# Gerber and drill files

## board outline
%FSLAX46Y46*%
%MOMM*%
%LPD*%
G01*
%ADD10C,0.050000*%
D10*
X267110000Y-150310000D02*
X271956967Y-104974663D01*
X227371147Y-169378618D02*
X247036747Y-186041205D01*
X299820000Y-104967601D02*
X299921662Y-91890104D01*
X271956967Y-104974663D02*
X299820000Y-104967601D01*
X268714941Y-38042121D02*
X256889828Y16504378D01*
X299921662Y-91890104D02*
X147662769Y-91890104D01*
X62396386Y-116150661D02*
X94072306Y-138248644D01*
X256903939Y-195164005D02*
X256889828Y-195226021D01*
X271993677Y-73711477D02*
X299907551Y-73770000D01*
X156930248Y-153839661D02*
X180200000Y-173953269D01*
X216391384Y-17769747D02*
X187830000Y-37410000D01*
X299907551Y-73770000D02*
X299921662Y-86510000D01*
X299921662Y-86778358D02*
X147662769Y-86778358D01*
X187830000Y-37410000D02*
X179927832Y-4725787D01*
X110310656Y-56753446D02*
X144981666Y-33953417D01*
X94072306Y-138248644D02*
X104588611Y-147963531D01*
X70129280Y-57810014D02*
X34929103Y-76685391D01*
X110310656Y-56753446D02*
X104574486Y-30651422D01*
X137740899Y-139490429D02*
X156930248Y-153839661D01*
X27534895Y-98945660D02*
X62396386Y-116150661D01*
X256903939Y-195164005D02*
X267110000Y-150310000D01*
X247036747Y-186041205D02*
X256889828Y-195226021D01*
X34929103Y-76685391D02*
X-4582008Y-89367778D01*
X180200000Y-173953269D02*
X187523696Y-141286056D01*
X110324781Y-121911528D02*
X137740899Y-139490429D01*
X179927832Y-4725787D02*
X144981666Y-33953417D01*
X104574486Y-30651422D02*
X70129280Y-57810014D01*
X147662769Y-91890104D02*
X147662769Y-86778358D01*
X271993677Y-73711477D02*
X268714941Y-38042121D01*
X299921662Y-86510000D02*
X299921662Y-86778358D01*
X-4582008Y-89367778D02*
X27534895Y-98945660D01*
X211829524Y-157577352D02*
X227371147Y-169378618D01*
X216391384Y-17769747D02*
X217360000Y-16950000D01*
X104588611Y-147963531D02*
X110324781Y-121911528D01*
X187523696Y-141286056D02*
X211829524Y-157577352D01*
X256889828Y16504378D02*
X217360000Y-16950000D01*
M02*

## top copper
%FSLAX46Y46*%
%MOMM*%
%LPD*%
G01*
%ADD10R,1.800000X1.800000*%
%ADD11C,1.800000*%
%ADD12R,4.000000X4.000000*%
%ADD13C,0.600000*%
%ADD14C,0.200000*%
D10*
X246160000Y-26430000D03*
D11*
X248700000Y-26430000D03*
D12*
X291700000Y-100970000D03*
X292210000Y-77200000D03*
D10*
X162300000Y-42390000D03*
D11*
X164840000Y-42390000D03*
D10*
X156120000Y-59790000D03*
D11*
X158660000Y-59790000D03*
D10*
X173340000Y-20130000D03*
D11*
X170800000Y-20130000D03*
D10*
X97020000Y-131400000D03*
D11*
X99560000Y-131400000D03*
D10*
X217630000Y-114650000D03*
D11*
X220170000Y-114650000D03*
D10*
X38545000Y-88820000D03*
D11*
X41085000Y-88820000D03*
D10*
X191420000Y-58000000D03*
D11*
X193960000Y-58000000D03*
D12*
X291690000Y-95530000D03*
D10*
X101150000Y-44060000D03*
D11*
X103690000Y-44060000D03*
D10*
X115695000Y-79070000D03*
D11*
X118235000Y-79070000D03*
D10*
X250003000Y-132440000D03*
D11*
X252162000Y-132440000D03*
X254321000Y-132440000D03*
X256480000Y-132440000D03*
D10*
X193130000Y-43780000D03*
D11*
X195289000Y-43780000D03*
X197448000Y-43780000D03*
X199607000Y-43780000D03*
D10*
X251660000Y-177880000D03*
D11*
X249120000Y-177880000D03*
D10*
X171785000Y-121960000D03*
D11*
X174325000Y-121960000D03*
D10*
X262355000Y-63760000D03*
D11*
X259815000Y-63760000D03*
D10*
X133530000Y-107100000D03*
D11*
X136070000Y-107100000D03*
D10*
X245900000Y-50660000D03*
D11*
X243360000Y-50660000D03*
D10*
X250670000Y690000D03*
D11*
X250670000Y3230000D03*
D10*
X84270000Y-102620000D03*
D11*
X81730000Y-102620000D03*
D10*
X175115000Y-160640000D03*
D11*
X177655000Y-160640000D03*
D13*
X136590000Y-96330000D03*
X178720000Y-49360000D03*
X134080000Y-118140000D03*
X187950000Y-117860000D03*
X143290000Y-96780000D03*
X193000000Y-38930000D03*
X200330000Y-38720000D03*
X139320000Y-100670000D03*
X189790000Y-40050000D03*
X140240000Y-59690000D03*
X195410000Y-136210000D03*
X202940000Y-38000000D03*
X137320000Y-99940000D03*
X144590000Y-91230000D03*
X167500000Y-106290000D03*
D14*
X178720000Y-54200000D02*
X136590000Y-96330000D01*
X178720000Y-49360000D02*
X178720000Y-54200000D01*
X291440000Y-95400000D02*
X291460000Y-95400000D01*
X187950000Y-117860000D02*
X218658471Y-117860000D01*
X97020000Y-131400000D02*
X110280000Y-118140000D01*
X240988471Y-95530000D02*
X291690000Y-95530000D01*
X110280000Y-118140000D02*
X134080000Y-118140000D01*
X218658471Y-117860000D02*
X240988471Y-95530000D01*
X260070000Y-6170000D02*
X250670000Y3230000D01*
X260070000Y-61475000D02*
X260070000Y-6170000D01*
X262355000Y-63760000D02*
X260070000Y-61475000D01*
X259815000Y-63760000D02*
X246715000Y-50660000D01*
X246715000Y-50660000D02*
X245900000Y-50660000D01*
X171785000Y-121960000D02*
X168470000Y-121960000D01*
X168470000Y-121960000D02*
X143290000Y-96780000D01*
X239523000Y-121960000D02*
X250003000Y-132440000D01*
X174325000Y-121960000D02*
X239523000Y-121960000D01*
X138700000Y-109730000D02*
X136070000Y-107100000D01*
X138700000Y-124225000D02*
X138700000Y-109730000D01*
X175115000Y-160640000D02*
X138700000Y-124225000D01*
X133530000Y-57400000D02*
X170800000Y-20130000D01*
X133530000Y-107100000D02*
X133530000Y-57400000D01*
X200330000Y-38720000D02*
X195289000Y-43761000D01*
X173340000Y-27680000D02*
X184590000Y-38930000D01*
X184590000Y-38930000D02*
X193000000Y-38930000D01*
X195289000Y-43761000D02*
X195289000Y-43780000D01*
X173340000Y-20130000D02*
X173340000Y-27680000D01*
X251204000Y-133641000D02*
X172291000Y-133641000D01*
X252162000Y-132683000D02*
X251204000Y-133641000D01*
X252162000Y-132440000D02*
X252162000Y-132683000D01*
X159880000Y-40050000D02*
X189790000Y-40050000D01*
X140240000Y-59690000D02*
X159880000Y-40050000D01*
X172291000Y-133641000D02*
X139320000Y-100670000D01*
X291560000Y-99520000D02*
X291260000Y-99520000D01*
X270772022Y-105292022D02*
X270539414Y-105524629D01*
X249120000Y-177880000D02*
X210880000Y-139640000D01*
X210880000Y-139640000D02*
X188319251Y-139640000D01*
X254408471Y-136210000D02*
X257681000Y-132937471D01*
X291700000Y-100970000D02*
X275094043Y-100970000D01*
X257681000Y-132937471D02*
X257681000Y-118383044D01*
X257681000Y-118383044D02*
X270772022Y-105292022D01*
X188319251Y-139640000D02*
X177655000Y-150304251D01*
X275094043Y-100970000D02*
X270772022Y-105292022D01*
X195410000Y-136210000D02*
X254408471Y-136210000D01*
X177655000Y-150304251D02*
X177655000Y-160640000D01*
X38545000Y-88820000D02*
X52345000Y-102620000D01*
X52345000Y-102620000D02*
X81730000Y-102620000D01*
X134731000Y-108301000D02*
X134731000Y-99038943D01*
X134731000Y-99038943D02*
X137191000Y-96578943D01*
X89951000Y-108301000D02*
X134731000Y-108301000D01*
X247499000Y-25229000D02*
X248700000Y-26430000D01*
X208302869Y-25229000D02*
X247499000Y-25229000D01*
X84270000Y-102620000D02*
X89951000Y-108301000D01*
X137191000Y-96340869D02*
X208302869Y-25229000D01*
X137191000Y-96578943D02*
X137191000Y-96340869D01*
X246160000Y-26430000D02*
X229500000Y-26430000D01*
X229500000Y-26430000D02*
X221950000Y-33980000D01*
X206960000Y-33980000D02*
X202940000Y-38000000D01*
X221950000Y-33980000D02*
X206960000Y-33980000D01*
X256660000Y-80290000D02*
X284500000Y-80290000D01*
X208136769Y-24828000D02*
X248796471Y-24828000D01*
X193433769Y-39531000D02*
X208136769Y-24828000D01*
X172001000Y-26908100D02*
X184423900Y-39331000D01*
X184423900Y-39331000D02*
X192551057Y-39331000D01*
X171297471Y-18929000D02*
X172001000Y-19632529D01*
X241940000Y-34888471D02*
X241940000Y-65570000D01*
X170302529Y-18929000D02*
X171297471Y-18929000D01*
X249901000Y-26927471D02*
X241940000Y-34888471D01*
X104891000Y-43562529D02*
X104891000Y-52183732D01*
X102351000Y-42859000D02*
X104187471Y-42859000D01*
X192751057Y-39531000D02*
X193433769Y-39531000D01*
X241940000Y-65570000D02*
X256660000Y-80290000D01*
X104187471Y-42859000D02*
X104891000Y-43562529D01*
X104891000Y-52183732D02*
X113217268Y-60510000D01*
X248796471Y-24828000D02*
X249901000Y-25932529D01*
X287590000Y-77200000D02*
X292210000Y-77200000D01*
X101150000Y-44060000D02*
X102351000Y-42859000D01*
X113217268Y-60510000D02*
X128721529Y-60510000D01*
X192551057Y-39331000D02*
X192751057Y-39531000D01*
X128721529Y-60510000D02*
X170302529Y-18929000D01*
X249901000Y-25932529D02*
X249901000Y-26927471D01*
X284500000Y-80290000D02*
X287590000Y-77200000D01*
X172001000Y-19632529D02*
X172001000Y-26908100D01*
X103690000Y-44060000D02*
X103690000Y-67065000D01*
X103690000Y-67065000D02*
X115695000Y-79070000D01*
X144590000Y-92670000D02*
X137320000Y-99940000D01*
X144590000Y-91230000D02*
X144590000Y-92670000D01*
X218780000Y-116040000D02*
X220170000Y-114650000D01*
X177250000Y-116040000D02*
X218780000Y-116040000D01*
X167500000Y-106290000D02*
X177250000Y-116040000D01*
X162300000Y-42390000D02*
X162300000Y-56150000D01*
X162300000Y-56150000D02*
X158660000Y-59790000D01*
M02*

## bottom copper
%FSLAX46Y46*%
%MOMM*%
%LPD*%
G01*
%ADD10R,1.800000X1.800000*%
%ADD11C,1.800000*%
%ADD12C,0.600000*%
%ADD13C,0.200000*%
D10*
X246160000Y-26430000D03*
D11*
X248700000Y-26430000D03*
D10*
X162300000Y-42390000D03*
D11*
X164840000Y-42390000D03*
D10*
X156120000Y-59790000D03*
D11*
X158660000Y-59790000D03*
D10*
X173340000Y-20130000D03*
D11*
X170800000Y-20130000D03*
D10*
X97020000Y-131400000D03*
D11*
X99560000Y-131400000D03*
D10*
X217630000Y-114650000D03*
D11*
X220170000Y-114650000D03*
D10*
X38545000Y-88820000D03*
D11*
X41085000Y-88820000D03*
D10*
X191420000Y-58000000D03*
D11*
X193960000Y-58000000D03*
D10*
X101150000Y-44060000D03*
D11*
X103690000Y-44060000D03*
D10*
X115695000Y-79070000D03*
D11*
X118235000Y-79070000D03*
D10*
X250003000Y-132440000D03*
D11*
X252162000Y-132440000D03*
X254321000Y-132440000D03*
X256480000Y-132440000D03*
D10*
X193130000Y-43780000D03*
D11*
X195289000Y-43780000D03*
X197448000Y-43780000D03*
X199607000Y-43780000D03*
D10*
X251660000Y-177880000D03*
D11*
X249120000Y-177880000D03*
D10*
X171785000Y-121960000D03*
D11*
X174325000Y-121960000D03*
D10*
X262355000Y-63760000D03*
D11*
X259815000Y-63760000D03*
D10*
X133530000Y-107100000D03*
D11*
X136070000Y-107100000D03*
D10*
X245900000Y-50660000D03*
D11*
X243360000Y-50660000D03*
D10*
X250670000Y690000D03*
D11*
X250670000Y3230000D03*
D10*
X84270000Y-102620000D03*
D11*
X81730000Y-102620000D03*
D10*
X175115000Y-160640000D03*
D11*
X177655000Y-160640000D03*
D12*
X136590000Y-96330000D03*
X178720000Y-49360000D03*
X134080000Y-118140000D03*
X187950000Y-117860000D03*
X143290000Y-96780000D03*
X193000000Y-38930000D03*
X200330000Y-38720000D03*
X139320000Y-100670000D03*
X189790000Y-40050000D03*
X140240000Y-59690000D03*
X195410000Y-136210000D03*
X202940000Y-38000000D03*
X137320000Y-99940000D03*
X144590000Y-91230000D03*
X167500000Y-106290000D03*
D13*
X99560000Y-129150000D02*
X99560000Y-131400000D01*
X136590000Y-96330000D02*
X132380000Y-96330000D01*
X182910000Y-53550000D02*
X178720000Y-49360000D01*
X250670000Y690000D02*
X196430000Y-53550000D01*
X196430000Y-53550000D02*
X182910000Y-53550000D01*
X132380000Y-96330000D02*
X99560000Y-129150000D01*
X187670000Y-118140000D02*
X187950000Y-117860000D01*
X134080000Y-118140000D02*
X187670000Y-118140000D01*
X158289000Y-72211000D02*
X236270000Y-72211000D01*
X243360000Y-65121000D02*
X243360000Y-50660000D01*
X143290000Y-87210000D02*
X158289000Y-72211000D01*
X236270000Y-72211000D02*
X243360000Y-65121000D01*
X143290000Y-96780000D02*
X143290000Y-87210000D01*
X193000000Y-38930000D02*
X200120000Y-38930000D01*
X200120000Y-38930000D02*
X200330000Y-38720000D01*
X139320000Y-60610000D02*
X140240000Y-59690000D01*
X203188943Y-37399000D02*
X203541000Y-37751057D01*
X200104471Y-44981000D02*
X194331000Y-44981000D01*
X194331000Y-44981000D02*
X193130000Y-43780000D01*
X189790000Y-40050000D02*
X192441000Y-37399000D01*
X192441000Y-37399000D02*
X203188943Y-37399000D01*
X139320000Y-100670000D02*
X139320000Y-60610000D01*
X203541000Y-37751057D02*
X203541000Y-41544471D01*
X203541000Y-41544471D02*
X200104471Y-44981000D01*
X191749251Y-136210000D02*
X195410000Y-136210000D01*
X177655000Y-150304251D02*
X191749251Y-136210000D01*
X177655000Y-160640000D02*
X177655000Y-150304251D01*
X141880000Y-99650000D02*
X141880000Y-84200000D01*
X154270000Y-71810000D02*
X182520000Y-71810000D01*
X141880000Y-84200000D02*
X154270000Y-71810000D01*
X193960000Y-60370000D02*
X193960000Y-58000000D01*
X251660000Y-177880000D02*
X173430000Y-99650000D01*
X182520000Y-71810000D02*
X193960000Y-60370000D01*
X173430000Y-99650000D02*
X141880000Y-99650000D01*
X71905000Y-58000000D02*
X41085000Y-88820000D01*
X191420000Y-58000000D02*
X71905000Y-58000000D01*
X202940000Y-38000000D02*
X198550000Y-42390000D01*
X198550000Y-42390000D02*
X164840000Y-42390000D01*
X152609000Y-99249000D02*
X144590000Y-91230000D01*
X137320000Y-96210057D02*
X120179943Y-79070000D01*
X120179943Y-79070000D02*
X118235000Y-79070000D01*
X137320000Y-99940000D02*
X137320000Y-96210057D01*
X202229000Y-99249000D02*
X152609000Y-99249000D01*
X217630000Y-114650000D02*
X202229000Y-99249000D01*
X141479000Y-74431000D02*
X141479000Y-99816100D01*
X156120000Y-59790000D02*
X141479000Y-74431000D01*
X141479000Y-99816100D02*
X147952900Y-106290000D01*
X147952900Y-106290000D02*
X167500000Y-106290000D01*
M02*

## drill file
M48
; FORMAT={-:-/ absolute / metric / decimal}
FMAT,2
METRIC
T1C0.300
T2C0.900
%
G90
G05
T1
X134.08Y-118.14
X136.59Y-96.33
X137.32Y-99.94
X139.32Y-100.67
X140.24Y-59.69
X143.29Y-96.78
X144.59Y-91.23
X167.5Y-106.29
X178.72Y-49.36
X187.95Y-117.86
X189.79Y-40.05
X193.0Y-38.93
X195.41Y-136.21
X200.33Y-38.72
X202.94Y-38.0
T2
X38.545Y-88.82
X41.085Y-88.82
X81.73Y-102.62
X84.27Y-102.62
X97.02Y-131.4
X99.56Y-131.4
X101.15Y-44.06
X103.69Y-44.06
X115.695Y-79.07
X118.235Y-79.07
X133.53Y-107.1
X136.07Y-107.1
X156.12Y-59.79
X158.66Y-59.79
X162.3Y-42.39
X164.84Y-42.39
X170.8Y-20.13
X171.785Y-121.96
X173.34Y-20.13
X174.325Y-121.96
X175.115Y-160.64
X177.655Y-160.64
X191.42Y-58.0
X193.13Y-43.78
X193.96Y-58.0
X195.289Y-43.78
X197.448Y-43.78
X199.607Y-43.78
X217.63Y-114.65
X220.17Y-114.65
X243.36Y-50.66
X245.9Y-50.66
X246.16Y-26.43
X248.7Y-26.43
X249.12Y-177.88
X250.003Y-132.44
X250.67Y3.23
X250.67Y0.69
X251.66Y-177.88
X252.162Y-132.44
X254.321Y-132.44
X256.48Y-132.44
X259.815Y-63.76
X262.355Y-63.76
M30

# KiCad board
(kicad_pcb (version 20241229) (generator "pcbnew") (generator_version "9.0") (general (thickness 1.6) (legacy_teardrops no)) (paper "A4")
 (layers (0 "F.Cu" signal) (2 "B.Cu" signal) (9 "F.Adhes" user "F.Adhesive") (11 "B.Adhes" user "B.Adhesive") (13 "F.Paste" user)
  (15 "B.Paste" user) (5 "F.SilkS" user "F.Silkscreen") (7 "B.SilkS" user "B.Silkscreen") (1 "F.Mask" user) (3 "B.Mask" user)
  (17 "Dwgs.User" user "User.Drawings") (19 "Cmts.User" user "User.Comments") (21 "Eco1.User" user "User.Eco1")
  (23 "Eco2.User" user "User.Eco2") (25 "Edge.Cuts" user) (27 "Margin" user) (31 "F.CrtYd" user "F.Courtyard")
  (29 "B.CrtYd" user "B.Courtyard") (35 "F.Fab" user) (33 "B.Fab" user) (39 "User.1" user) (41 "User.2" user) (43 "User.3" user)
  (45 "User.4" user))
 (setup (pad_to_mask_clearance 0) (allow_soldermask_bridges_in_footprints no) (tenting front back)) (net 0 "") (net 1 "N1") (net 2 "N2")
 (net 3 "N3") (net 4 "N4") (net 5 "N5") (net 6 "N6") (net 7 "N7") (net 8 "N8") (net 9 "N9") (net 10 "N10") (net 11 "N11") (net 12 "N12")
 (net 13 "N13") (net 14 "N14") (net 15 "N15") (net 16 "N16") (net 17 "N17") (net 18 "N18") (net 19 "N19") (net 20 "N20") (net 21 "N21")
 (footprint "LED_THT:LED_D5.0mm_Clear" (layer "F.Cu") (at 246.16 26.43)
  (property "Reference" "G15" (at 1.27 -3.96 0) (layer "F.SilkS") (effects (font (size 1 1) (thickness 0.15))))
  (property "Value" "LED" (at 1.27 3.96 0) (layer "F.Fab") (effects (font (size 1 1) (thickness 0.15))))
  (pad "1" thru_hole rect (at 0 0) (size 1.8 1.8) (drill 0.9) (layers "*.Cu" "*.Mask") (remove_unused_layers no) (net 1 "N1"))
  (pad "2" thru_hole circle (at 2.54 0) (size 1.8 1.8) (drill 0.9) (layers "*.Cu" "*.Mask") (remove_unused_layers no) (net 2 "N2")))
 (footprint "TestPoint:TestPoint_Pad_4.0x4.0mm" (layer "F.Cu") (at 291.7 100.97)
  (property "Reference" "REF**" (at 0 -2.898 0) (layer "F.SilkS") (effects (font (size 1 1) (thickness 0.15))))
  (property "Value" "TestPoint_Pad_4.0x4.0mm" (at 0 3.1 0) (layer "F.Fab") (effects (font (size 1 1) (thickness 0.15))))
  (pad "1" smd rect (at 0 0) (size 4 4) (layers "F.Cu" "F.Mask") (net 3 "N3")))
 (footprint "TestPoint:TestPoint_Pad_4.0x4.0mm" (layer "F.Cu") (at 292.21 77.2)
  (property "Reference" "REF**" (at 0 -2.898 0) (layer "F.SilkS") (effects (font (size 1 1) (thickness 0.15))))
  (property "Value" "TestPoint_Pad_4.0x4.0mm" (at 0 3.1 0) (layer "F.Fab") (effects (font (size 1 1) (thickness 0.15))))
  (pad "1" smd rect (at 0 0) (size 4 4) (layers "F.Cu" "F.Mask") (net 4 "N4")))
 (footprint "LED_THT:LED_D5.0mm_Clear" (layer "F.Cu") (at 162.3 42.39)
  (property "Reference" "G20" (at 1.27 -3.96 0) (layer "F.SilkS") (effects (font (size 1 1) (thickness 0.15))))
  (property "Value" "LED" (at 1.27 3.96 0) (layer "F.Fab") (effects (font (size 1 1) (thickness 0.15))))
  (pad "1" thru_hole rect (at 0 0) (size 1.8 1.8) (drill 0.9) (layers "*.Cu" "*.Mask") (remove_unused_layers no) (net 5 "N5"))
  (pad "2" thru_hole circle (at 2.54 0) (size 1.8 1.8) (drill 0.9) (layers "*.Cu" "*.Mask") (remove_unused_layers no) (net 1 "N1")))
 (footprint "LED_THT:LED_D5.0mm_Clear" (layer "F.Cu") (at 156.12 59.79)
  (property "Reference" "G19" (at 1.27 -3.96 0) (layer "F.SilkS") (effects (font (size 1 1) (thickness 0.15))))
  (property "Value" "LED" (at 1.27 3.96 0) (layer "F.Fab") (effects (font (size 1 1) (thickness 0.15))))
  (pad "1" thru_hole rect (at 0 0) (size 1.8 1.8) (drill 0.9) (layers "*.Cu" "*.Mask") (remove_unused_layers no) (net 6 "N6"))
  (pad "2" thru_hole circle (at 2.54 0) (size 1.8 1.8) (drill 0.9) (layers "*.Cu" "*.Mask") (remove_unused_layers no) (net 5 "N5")))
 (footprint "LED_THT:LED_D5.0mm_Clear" (layer "F.Cu") (at 173.34 20.13 180)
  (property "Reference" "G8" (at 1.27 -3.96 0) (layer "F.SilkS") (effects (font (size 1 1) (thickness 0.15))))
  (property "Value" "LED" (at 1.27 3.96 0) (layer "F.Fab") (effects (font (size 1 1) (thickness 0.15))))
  (pad "1" thru_hole rect (at 0 0 180) (size 1.8 1.8) (drill 0.9) (layers "*.Cu" "*.Mask") (remove_unused_layers no) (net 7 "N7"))
  (pad "2" thru_hole circle (at 2.54 0 180) (size 1.8 1.8) (drill 0.9) (layers "*.Cu" "*.Mask") (remove_unused_layers no) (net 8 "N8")))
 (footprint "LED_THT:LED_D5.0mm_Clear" (layer "F.Cu") (at 97.02 131.4)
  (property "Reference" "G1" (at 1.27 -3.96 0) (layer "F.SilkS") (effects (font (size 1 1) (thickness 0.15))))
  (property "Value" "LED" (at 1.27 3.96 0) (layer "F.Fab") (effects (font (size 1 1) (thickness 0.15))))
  (pad "1" thru_hole rect (at 0 0) (size 1.8 1.8) (drill 0.9) (layers "*.Cu" "*.Mask") (remove_unused_layers no) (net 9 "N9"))
  (pad "2" thru_hole circle (at 2.54 0) (size 1.8 1.8) (drill 0.9) (layers "*.Cu" "*.Mask") (remove_unused_layers no) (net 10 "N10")))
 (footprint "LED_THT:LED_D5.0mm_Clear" (layer "F.Cu") (at 217.63 114.65)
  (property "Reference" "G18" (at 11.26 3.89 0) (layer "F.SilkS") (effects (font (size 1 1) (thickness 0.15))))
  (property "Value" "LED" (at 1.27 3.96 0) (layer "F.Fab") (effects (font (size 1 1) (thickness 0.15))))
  (pad "1" thru_hole rect (at 0 0) (size 1.8 1.8) (drill 0.9) (layers "*.Cu" "*.Mask") (remove_unused_layers no) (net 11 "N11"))
  (pad "2" thru_hole circle (at 2.54 0) (size 1.8 1.8) (drill 0.9) (layers "*.Cu" "*.Mask") (remove_unused_layers no) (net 6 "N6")))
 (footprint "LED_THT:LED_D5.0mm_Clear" (layer "F.Cu") (at 38.545 88.82)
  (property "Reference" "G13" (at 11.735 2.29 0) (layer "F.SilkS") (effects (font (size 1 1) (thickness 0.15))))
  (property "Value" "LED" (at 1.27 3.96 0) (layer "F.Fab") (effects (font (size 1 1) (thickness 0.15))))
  (pad "1" thru_hole rect (at 0 0) (size 1.8 1.8) (drill 0.9) (layers "*.Cu" "*.Mask") (remove_unused_layers no) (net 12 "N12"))
  (pad "2" thru_hole circle (at 2.54 0) (size 1.8 1.8) (drill 0.9) (layers "*.Cu" "*.Mask") (remove_unused_layers no) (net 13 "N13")))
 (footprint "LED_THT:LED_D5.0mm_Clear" (layer "F.Cu") (at 191.42 58)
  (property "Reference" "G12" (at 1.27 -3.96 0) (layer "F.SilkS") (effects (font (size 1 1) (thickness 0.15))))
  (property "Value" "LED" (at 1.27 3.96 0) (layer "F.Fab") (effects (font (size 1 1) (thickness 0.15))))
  (pad "1" thru_hole rect (at 0 0) (size 1.8 1.8) (drill 0.9) (layers "*.Cu" "*.Mask") (remove_unused_layers no) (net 13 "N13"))
  (pad "2" thru_hole circle (at 2.54 0) (size 1.8 1.8) (drill 0.9) (layers "*.Cu" "*.Mask") (remove_unused_layers no) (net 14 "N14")))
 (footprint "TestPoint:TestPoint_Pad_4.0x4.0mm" (layer "F.Cu") (at 291.69 95.53)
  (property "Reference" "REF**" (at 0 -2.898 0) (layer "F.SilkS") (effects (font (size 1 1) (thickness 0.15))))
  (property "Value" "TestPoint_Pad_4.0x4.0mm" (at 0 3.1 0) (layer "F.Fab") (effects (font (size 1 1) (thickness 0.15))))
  (pad "1" smd rect (at 0 0) (size 4 4) (layers "F.Cu" "F.Mask") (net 9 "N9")))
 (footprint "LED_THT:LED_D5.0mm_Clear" (layer "F.Cu") (at 101.15 44.06)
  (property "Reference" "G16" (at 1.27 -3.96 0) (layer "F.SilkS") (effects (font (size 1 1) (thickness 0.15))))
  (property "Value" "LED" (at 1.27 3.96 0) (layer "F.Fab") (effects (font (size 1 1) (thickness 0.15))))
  (pad "1" thru_hole rect (at 0 0) (size 1.8 1.8) (drill 0.9) (layers "*.Cu" "*.Mask") (remove_unused_layers no) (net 4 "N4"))
  (pad "2" thru_hole circle (at 2.54 0) (size 1.8 1.8) (drill 0.9) (layers "*.Cu" "*.Mask") (remove_unused_layers no) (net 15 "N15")))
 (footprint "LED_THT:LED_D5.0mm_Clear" (layer "F.Cu") (at 115.695 79.07)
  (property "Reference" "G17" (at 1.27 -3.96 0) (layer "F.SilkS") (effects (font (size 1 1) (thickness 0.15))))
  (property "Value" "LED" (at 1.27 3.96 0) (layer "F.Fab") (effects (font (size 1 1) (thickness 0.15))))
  (pad "1" thru_hole rect (at 0 0) (size 1.8 1.8) (drill 0.9) (layers "*.Cu" "*.Mask") (remove_unused_layers no) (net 15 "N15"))
  (pad "2" thru_hole circle (at 2.54 0) (size 1.8 1.8) (drill 0.9) (layers "*.Cu" "*.Mask") (remove_unused_layers no) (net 11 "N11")))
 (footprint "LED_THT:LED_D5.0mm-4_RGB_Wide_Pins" (layer "F.Cu") (at 250.003 132.44)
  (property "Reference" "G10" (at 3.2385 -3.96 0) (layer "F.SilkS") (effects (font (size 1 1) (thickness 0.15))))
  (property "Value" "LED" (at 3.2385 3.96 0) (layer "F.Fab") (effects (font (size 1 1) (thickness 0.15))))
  (pad "1" thru_hole rect (at 0 0) (size 1.8 1.8) (drill 0.9) (layers "*.Cu" "*.Mask") (remove_unused_layers no) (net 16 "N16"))
  (pad "2" thru_hole circle (at 2.159 0) (size 1.8 1.8) (drill 0.9) (layers "*.Cu" "*.Mask") (remove_unused_layers no) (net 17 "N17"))
  (pad "3" thru_hole circle (at 4.318 0) (size 1.8 1.8) (drill 0.9) (layers "*.Cu" "*.Mask") (remove_unused_layers no))
  (pad "4" thru_hole circle (at 6.477 0) (size 1.8 1.8) (drill 0.9) (layers "*.Cu" "*.Mask") (remove_unused_layers no)))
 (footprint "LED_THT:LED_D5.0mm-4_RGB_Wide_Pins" (layer "F.Cu") (at 193.13 43.78)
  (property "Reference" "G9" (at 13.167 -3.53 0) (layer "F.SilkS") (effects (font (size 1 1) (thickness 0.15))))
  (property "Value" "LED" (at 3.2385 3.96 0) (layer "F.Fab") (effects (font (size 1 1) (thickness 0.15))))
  (pad "1" thru_hole rect (at 0 0) (size 1.8 1.8) (drill 0.9) (layers "*.Cu" "*.Mask") (remove_unused_layers no) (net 17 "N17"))
  (pad "2" thru_hole circle (at 2.159 0) (size 1.8 1.8) (drill 0.9) (layers "*.Cu" "*.Mask") (remove_unused_layers no) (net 7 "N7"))
  (pad "3" thru_hole circle (at 4.318 0) (size 1.8 1.8) (drill 0.9) (layers "*.Cu" "*.Mask") (remove_unused_layers no))
  (pad "4" thru_hole circle (at 6.477 0) (size 1.8 1.8) (drill 0.9) (layers "*.Cu" "*.Mask") (remove_unused_layers no)))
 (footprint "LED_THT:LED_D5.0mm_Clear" (layer "F.Cu") (at 251.66 177.88 180)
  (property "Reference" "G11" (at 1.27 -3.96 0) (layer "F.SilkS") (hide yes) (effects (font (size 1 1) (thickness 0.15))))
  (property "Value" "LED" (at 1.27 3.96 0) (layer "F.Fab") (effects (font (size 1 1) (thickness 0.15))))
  (pad "1" thru_hole rect (at 0 0 180) (size 1.8 1.8) (drill 0.9) (layers "*.Cu" "*.Mask") (remove_unused_layers no) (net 14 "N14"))
  (pad "2" thru_hole circle (at 2.54 0 180) (size 1.8 1.8) (drill 0.9) (layers "*.Cu" "*.Mask") (remove_unused_layers no) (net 3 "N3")))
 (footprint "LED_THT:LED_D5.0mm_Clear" (layer "F.Cu") (at 171.785 121.96)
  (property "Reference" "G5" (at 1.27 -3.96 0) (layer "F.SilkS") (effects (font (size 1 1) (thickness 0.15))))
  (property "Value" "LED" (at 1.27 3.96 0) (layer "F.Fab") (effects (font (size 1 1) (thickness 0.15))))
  (pad "1" thru_hole rect (at 0 0) (size 1.8 1.8) (drill 0.9) (layers "*.Cu" "*.Mask") (remove_unused_layers no) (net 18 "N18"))
  (pad "2" thru_hole circle (at 2.54 0) (size 1.8 1.8) (drill 0.9) (layers "*.Cu" "*.Mask") (remove_unused_layers no) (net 16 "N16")))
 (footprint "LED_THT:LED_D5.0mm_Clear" (layer "F.Cu") (at 262.355 63.76 180)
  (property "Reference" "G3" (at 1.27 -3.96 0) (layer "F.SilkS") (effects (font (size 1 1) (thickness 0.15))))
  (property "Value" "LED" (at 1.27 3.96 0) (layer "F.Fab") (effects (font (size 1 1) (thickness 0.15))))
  (pad "1" thru_hole rect (at 0 0 180) (size 1.8 1.8) (drill 0.9) (layers "*.Cu" "*.Mask") (remove_unused_layers no) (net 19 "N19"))
  (pad "2" thru_hole circle (at 2.54 0 180) (size 1.8 1.8) (drill 0.9) (layers "*.Cu" "*.Mask") (remove_unused_layers no) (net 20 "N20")))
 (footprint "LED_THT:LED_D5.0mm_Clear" (layer "F.Cu") (at 133.53 107.1)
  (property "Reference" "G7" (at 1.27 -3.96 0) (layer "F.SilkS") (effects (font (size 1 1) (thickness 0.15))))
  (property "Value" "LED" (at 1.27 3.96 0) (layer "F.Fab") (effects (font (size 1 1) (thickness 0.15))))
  (pad "1" thru_hole rect (at 0 0) (size 1.8 1.8) (drill 0.9) (layers "*.Cu" "*.Mask") (remove_unused_layers no) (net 8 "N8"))
  (pad "2" thru_hole circle (at 2.54 0) (size 1.8 1.8) (drill 0.9) (layers "*.Cu" "*.Mask") (remove_unused_layers no) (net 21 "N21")))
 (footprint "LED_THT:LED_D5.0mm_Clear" (layer "F.Cu") (at 245.9 50.66 180)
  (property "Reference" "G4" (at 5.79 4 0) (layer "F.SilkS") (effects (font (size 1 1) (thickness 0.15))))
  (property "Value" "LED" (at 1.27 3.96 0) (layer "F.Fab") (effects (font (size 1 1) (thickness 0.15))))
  (pad "1" thru_hole rect (at 0 0 180) (size 1.8 1.8) (drill 0.9) (layers "*.Cu" "*.Mask") (remove_unused_layers no) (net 20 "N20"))
  (pad "2" thru_hole circle (at 2.54 0 180) (size 1.8 1.8) (drill 0.9) (layers "*.Cu" "*.Mask") (remove_unused_layers no) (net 18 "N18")))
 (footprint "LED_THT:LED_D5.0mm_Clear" (layer "F.Cu") (at 250.67 -0.69 90)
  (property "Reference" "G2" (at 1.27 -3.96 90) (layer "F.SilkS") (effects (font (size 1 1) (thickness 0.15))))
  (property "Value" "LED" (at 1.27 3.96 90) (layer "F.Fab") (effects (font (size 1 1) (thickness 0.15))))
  (pad "1" thru_hole rect (at 0 0 90) (size 1.8 1.8) (drill 0.9) (layers "*.Cu" "*.Mask") (remove_unused_layers no) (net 10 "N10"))
  (pad "2" thru_hole circle (at 2.54 0 90) (size 1.8 1.8) (drill 0.9) (layers "*.Cu" "*.Mask") (remove_unused_layers no) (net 19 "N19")))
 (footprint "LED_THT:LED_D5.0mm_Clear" (layer "F.Cu") (at 84.27 102.62 180)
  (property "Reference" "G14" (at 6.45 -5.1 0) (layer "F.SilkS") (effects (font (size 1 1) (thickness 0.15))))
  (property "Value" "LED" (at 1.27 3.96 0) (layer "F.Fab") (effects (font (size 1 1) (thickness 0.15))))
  (pad "1" thru_hole rect (at 0 0 180) (size 1.8 1.8) (drill 0.9) (layers "*.Cu" "*.Mask") (remove_unused_layers no) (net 2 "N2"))
  (pad "2" thru_hole circle (at 2.54 0 180) (size 1.8 1.8) (drill 0.9) (layers "*.Cu" "*.Mask") (remove_unused_layers no) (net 12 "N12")))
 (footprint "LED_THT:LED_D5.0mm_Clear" (layer "F.Cu") (at 175.115 160.64)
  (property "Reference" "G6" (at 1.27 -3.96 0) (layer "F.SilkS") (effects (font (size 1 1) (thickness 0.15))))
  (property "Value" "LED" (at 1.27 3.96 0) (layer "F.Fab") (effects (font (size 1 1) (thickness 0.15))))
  (pad "1" thru_hole rect (at 0 0) (size 1.8 1.8) (drill 0.9) (layers "*.Cu" "*.Mask") (remove_unused_layers no) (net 21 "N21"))
  (pad "2" thru_hole circle (at 2.54 0) (size 1.8 1.8) (drill 0.9) (layers "*.Cu" "*.Mask") (remove_unused_layers no) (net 3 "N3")))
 (gr_line (start 267.11 150.31) (end 271.956967 104.974663) (stroke (width 0.05) (type default)) (layer "Edge.Cuts"))
 (gr_line (start 227.371147 169.378618) (end 247.036747 186.041205) (stroke (width 0.05) (type default)) (layer "Edge.Cuts"))
 (gr_line (start 299.82 104.967601) (end 299.921662 91.890104) (stroke (width 0.05) (type default)) (layer "Edge.Cuts"))
 (gr_line (start 271.956967 104.974663) (end 299.82 104.967601) (stroke (width 0.05) (type default)) (layer "Edge.Cuts"))
 (gr_line (start 268.714941 38.042121) (end 256.889828 -16.504378) (stroke (width 0.05) (type default)) (layer "Edge.Cuts"))
 (gr_line (start 299.921662 91.890104) (end 147.662769 91.890104) (stroke (width 0.05) (type default)) (layer "Edge.Cuts"))
 (gr_line (start 62.396386 116.150661) (end 94.072306 138.248644) (stroke (width 0.05) (type default)) (layer "Edge.Cuts"))
 (gr_line (start 256.903939 195.164005) (end 256.889828 195.226021) (stroke (width 0.05) (type default)) (layer "Edge.Cuts"))
 (gr_line (start 271.993677 73.711477) (end 299.907551 73.77) (stroke (width 0.05) (type default)) (layer "Edge.Cuts"))
 (gr_line (start 156.930248 153.839661) (end 180.2 173.953269) (stroke (width 0.05) (type default)) (layer "Edge.Cuts"))
 (gr_line (start 216.391384 17.769747) (end 187.83 37.41) (stroke (width 0.05) (type default)) (layer "Edge.Cuts"))
 (gr_line (start 299.907551 73.77) (end 299.921662 86.51) (stroke (width 0.05) (type default)) (layer "Edge.Cuts"))
 (gr_line (start 299.921662 86.778358) (end 147.662769 86.778358) (stroke (width 0.05) (type default)) (layer "Edge.Cuts"))
 (gr_line (start 187.83 37.41) (end 179.927832 4.725787) (stroke (width 0.05) (type default)) (layer "Edge.Cuts"))
 (gr_line (start 110.310656 56.753446) (end 144.981666 33.953417) (stroke (width 0.05) (type default)) (layer "Edge.Cuts"))
 (gr_line (start 94.072306 138.248644) (end 104.588611 147.963531) (stroke (width 0.05) (type default)) (layer "Edge.Cuts"))
 (gr_line (start 70.12928 57.810014) (end 34.929103 76.685391) (stroke (width 0.05) (type default)) (layer "Edge.Cuts"))
 (gr_line (start 110.310656 56.753446) (end 104.574486 30.651422) (stroke (width 0.05) (type default)) (layer "Edge.Cuts"))
 (gr_line (start 137.740899 139.490429) (end 156.930248 153.839661) (stroke (width 0.05) (type default)) (layer "Edge.Cuts"))
 (gr_line (start 27.534895 98.94566) (end 62.396386 116.150661) (stroke (width 0.05) (type default)) (layer "Edge.Cuts"))
 (gr_line (start 256.903939 195.164005) (end 267.11 150.31) (stroke (width 0.05) (type default)) (layer "Edge.Cuts"))
 (gr_line (start 247.036747 186.041205) (end 256.889828 195.226021) (stroke (width 0.05) (type default)) (layer "Edge.Cuts"))
 (gr_line (start 34.929103 76.685391) (end -4.582008 89.367778) (stroke (width 0.05) (type default)) (layer "Edge.Cuts"))
 (gr_line (start 180.2 173.953269) (end 187.523696 141.286056) (stroke (width 0.05) (type default)) (layer "Edge.Cuts"))
 (gr_line (start 110.324781 121.911528) (end 137.740899 139.490429) (stroke (width 0.05) (type default)) (layer "Edge.Cuts"))
 (gr_line (start 179.927832 4.725787) (end 144.981666 33.953417) (stroke (width 0.05) (type default)) (layer "Edge.Cuts"))
 (gr_line (start 104.574486 30.651422) (end 70.12928 57.810014) (stroke (width 0.05) (type default)) (layer "Edge.Cuts"))
 (gr_line (start 147.662769 91.890104) (end 147.662769 86.778358) (stroke (width 0.05) (type default)) (layer "Edge.Cuts"))
 (gr_line (start 271.993677 73.711477) (end 268.714941 38.042121) (stroke (width 0.05) (type default)) (layer "Edge.Cuts"))
 (gr_line (start 299.921662 86.51) (end 299.921662 86.778358) (stroke (width 0.05) (type default)) (layer "Edge.Cuts"))
 (gr_line (start -4.582008 89.367778) (end 27.534895 98.94566) (stroke (width 0.05) (type default)) (layer "Edge.Cuts"))
 (gr_line (start 211.829524 157.577352) (end 227.371147 169.378618) (stroke (width 0.05) (type default)) (layer "Edge.Cuts"))
 (gr_line (start 216.391384 17.769747) (end 217.36 16.95) (stroke (width 0.05) (type default)) (layer "Edge.Cuts"))
 (gr_line (start 104.588611 147.963531) (end 110.324781 121.911528) (stroke (width 0.05) (type default)) (layer "Edge.Cuts"))
 (gr_line (start 187.523696 141.286056) (end 211.829524 157.577352) (stroke (width 0.05) (type default)) (layer "Edge.Cuts"))
 (gr_line (start 256.889828 -16.504378) (end 217.36 16.95) (stroke (width 0.05) (type default)) (layer "Edge.Cuts"))
 (segment (start 178.72 54.2) (end 136.59 96.33) (width 0.2) (layer "F.Cu") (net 10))
 (segment (start 178.72 49.36) (end 178.72 54.2) (width 0.2) (layer "F.Cu") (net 10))
 (via (at 136.59 96.33) (size 0.6) (drill 0.3) (layers "F.Cu" "B.Cu") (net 10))
 (via (at 178.72 49.36) (size 0.6) (drill 0.3) (layers "F.Cu" "B.Cu") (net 10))
 (segment (start 99.56 129.15) (end 99.56 131.4) (width 0.2) (layer "B.Cu") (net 10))
 (segment (start 136.59 96.33) (end 132.38 96.33) (width 0.2) (layer "B.Cu") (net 10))
 (segment (start 182.91 53.55) (end 178.72 49.36) (width 0.2) (layer "B.Cu") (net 10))
 (segment (start 250.67 -0.69) (end 196.43 53.55) (width 0.2) (layer "B.Cu") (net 10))
 (segment (start 196.43 53.55) (end 182.91 53.55) (width 0.2) (layer "B.Cu") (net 10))
 (segment (start 132.38 96.33) (end 99.56 129.15) (width 0.2) (layer "B.Cu") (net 10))
 (segment (start 291.44 95.4) (end 291.46 95.4) (width 0.2) (layer "F.Cu") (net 9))
 (segment (start 187.95 117.86) (end 218.658471 117.86) (width 0.2) (layer "F.Cu") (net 9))
 (segment (start 97.02 131.4) (end 110.28 118.14) (width 0.2) (layer "F.Cu") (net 9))
 (segment (start 240.988471 95.53) (end 291.69 95.53) (width 0.2) (layer "F.Cu") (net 9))
 (segment (start 110.28 118.14) (end 134.08 118.14) (width 0.2) (layer "F.Cu") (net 9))
 (segment (start 218.658471 117.86) (end 240.988471 95.53) (width 0.2) (layer "F.Cu") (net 9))
 (via (at 134.08 118.14) (size 0.6) (drill 0.3) (layers "F.Cu" "B.Cu") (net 9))
 (via (at 187.95 117.86) (size 0.6) (drill 0.3) (layers "F.Cu" "B.Cu") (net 9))
 (segment (start 187.67 118.14) (end 187.95 117.86) (width 0.2) (layer "B.Cu") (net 9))
 (segment (start 134.08 118.14) (end 187.67 118.14) (width 0.2) (layer "B.Cu") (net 9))
 (segment (start 260.07 6.17) (end 250.67 -3.23) (width 0.2) (layer "F.Cu") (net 19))
 (segment (start 260.07 61.475) (end 260.07 6.17) (width 0.2) (layer "F.Cu") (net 19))
 (segment (start 262.355 63.76) (end 260.07 61.475) (width 0.2) (layer "F.Cu") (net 19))
 (segment (start 259.815 63.76) (end 246.715 50.66) (width 0.2) (layer "F.Cu") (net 20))
 (segment (start 246.715 50.66) (end 245.9 50.66) (width 0.2) (layer "F.Cu") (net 20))
 (segment (start 171.785 121.96) (end 168.47 121.96) (width 0.2) (layer "F.Cu") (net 18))
 (segment (start 168.47 121.96) (end 143.29 96.78) (width 0.2) (layer "F.Cu") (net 18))
 (via (at 143.29 96.78) (size 0.6) (drill 0.3) (layers "F.Cu" "B.Cu") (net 18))
 (segment (start 158.289 72.211) (end 236.27 72.211) (width 0.2) (layer "B.Cu") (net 18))
 (segment (start 243.36 65.121) (end 243.36 50.66) (width 0.2) (layer "B.Cu") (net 18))
 (segment (start 143.29 87.21) (end 158.289 72.211) (width 0.2) (layer "B.Cu") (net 18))
 (segment (start 236.27 72.211) (end 243.36 65.121) (width 0.2) (layer "B.Cu") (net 18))
 (segment (start 143.29 96.78) (end 143.29 87.21) (width 0.2) (layer "B.Cu") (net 18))
 (segment (start 239.523 121.96) (end 250.003 132.44) (width 0.2) (layer "F.Cu") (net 16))
 (segment (start 174.325 121.96) (end 239.523 121.96) (width 0.2) (layer "F.Cu") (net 16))
 (segment (start 138.7 109.73) (end 136.07 107.1) (width 0.2) (layer "F.Cu") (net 21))
 (segment (start 138.7 124.225) (end 138.7 109.73) (width 0.2) (layer "F.Cu") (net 21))
 (segment (start 175.115 160.64) (end 138.7 124.225) (width 0.2) (layer "F.Cu") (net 21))
 (segment (start 133.53 57.4) (end 170.8 20.13) (width 0.2) (layer "F.Cu") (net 8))
 (segment (start 133.53 107.1) (end 133.53 57.4) (width 0.2) (layer "F.Cu") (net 8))
 (segment (start 200.33 38.72) (end 195.289 43.761) (width 0.2) (layer "F.Cu") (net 7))
 (segment (start 173.34 27.68) (end 184.59 38.93) (width 0.2) (layer "F.Cu") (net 7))
 (segment (start 184.59 38.93) (end 193 38.93) (width 0.2) (layer "F.Cu") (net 7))
 (segment (start 195.289 43.761) (end 195.289 43.78) (width 0.2) (layer "F.Cu") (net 7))
 (segment (start 173.34 20.13) (end 173.34 27.68) (width 0.2) (layer "F.Cu") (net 7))
 (via (at 193 38.93) (size 0.6) (drill 0.3) (layers "F.Cu" "B.Cu") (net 7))
 (via (at 200.33 38.72) (size 0.6) (drill 0.3) (layers "F.Cu" "B.Cu") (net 7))
 (segment (start 193 38.93) (end 200.12 38.93) (width 0.2) (layer "B.Cu") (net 7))
 (segment (start 200.12 38.93) (end 200.33 38.72) (width 0.2) (layer "B.Cu") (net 7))
 (segment (start 251.204 133.641) (end 172.291 133.641) (width 0.2) (layer "F.Cu") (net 17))
 (segment (start 252.162 132.683) (end 251.204 133.641) (width 0.2) (layer "F.Cu") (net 17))
 (segment (start 252.162 132.44) (end 252.162 132.683) (width 0.2) (layer "F.Cu") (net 17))
 (segment (start 159.88 40.05) (end 189.79 40.05) (width 0.2) (layer "F.Cu") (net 17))
 (segment (start 140.24 59.69) (end 159.88 40.05) (width 0.2) (layer "F.Cu") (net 17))
 (segment (start 172.291 133.641) (end 139.32 100.67) (width 0.2) (layer "F.Cu") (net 17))
 (via (at 139.32 100.67) (size 0.6) (drill 0.3) (layers "F.Cu" "B.Cu") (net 17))
 (via (at 189.79 40.05) (size 0.6) (drill 0.3) (layers "F.Cu" "B.Cu") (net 17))
 (via (at 140.24 59.69) (size 0.6) (drill 0.3) (layers "F.Cu" "B.Cu") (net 17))
 (segment (start 139.32 60.61) (end 140.24 59.69) (width 0.2) (layer "B.Cu") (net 17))
 (segment (start 203.188943 37.399) (end 203.541 37.751057) (width 0.2) (layer "B.Cu") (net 17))
 (segment (start 200.104471 44.981) (end 194.331 44.981) (width 0.2) (layer "B.Cu") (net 17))
 (segment (start 194.331 44.981) (end 193.13 43.78) (width 0.2) (layer "B.Cu") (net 17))
 (segment (start 189.79 40.05) (end 192.441 37.399) (width 0.2) (layer "B.Cu") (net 17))
 (segment (start 192.441 37.399) (end 203.188943 37.399) (width 0.2) (layer "B.Cu") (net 17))
 (segment (start 139.32 100.67) (end 139.32 60.61) (width 0.2) (layer "B.Cu") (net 17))
 (segment (start 203.541 37.751057) (end 203.541 41.544471) (width 0.2) (layer "B.Cu") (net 17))
 (segment (start 203.541 41.544471) (end 200.104471 44.981) (width 0.2) (layer "B.Cu") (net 17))
 (segment (start 291.56 99.52) (end 291.26 99.52) (width 0.2) (layer "F.Cu") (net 3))
 (segment (start 270.772022 105.292022) (end 270.539414 105.524629) (width 0.2) (layer "F.Cu") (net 3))
 (segment (start 249.12 177.88) (end 210.88 139.64) (width 0.2) (layer "F.Cu") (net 3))
 (segment (start 210.88 139.64) (end 188.319251 139.64) (width 0.2) (layer "F.Cu") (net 3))
 (segment (start 254.408471 136.21) (end 257.681 132.937471) (width 0.2) (layer "F.Cu") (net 3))
 (segment (start 291.7 100.97) (end 275.094043 100.97) (width 0.2) (layer "F.Cu") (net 3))
 (segment (start 257.681 132.937471) (end 257.681 118.383044) (width 0.2) (layer "F.Cu") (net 3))
 (segment (start 257.681 118.383044) (end 270.772022 105.292022) (width 0.2) (layer "F.Cu") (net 3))
 (segment (start 188.319251 139.64) (end 177.655 150.304251) (width 0.2) (layer "F.Cu") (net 3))
 (segment (start 275.094043 100.97) (end 270.772022 105.292022) (width 0.2) (layer "F.Cu") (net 3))
 (segment (start 195.41 136.21) (end 254.408471 136.21) (width 0.2) (layer "F.Cu") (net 3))
 (segment (start 177.655 150.304251) (end 177.655 160.64) (width 0.2) (layer "F.Cu") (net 3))
 (via (at 195.41 136.21) (size 0.6) (drill 0.3) (layers "F.Cu" "B.Cu") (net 3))
 (segment (start 191.749251 136.21) (end 195.41 136.21) (width 0.2) (layer "B.Cu") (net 3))
 (segment (start 177.655 150.304251) (end 191.749251 136.21) (width 0.2) (layer "B.Cu") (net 3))
 (segment (start 177.655 160.64) (end 177.655 150.304251) (width 0.2) (layer "B.Cu") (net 3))
 (segment (start 141.88 99.65) (end 141.88 84.2) (width 0.2) (layer "B.Cu") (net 14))
 (segment (start 154.27 71.81) (end 182.52 71.81) (width 0.2) (layer "B.Cu") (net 14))
 (segment (start 141.88 84.2) (end 154.27 71.81) (width 0.2) (layer "B.Cu") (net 14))
 (segment (start 193.96 60.37) (end 193.96 58) (width 0.2) (layer "B.Cu") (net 14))
 (segment (start 251.66 177.88) (end 173.43 99.65) (width 0.2) (layer "B.Cu") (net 14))
 (segment (start 182.52 71.81) (end 193.96 60.37) (width 0.2) (layer "B.Cu") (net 14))
 (segment (start 173.43 99.65) (end 141.88 99.65) (width 0.2) (layer "B.Cu") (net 14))
 (segment (start 71.905 58) (end 41.085 88.82) (width 0.2) (layer "B.Cu") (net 13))
 (segment (start 191.42 58) (end 71.905 58) (width 0.2) (layer "B.Cu") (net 13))
 (segment (start 38.545 88.82) (end 52.345 102.62) (width 0.2) (layer "F.Cu") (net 12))
 (segment (start 52.345 102.62) (end 81.73 102.62) (width 0.2) (layer "F.Cu") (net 12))
 (segment (start 134.731 108.301) (end 134.731 99.038943) (width 0.2) (layer "F.Cu") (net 2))
 (segment (start 134.731 99.038943) (end 137.191 96.578943) (width 0.2) (layer "F.Cu") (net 2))
 (segment (start 89.951 108.301) (end 134.731 108.301) (width 0.2) (layer "F.Cu") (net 2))
 (segment (start 247.499 25.229) (end 248.7 26.43) (width 0.2) (layer "F.Cu") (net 2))
 (segment (start 208.302869 25.229) (end 247.499 25.229) (width 0.2) (layer "F.Cu") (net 2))
 (segment (start 84.27 102.62) (end 89.951 108.301) (width 0.2) (layer "F.Cu") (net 2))
 (segment (start 137.191 96.340869) (end 208.302869 25.229) (width 0.2) (layer "F.Cu") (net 2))
 (segment (start 137.191 96.578943) (end 137.191 96.340869) (width 0.2) (layer "F.Cu") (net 2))
 (segment (start 246.16 26.43) (end 229.5 26.43) (width 0.2) (layer "F.Cu") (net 1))
 (segment (start 229.5 26.43) (end 221.95 33.98) (width 0.2) (layer "F.Cu") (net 1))
 (segment (start 206.96 33.98) (end 202.94 38) (width 0.2) (layer "F.Cu") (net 1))
 (segment (start 221.95 33.98) (end 206.96 33.98) (width 0.2) (layer "F.Cu") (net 1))
 (via (at 202.94 38) (size 0.6) (drill 0.3) (layers "F.Cu" "B.Cu") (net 1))
 (segment (start 202.94 38) (end 198.55 42.39) (width 0.2) (layer "B.Cu") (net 1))
 (segment (start 198.55 42.39) (end 164.84 42.39) (width 0.2) (layer "B.Cu") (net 1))
 (segment (start 256.66 80.29) (end 284.5 80.29) (width 0.2) (layer "F.Cu") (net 4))
 (segment (start 208.136769 24.828) (end 248.796471 24.828) (width 0.2) (layer "F.Cu") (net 4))
 (segment (start 193.433769 39.531) (end 208.136769 24.828) (width 0.2) (layer "F.Cu") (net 4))
 (segment (start 172.001 26.9081) (end 184.4239 39.331) (width 0.2) (layer "F.Cu") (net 4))
 (segment (start 184.4239 39.331) (end 192.551057 39.331) (width 0.2) (layer "F.Cu") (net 4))
 (segment (start 171.297471 18.929) (end 172.001 19.632529) (width 0.2) (layer "F.Cu") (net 4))
 (segment (start 241.94 34.888471) (end 241.94 65.57) (width 0.2) (layer "F.Cu") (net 4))
 (segment (start 170.302529 18.929) (end 171.297471 18.929) (width 0.2) (layer "F.Cu") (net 4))
 (segment (start 249.901 26.927471) (end 241.94 34.888471) (width 0.2) (layer "F.Cu") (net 4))
 (segment (start 104.891 43.562529) (end 104.891 52.183732) (width 0.2) (layer "F.Cu") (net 4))
 (segment (start 102.351 42.859) (end 104.187471 42.859) (width 0.2) (layer "F.Cu") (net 4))
 (segment (start 192.751057 39.531) (end 193.433769 39.531) (width 0.2) (layer "F.Cu") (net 4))
 (segment (start 241.94 65.57) (end 256.66 80.29) (width 0.2) (layer "F.Cu") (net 4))
 (segment (start 104.187471 42.859) (end 104.891 43.562529) (width 0.2) (layer "F.Cu") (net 4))
 (segment (start 104.891 52.183732) (end 113.217268 60.51) (width 0.2) (layer "F.Cu") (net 4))
 (segment (start 248.796471 24.828) (end 249.901 25.932529) (width 0.2) (layer "F.Cu") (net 4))
 (segment (start 287.59 77.2) (end 292.21 77.2) (width 0.2) (layer "F.Cu") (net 4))
 (segment (start 101.15 44.06) (end 102.351 42.859) (width 0.2) (layer "F.Cu") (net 4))
 (segment (start 113.217268 60.51) (end 128.721529 60.51) (width 0.2) (layer "F.Cu") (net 4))
 (segment (start 192.551057 39.331) (end 192.751057 39.531) (width 0.2) (layer "F.Cu") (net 4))
 (segment (start 128.721529 60.51) (end 170.302529 18.929) (width 0.2) (layer "F.Cu") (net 4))
 (segment (start 249.901 25.932529) (end 249.901 26.927471) (width 0.2) (layer "F.Cu") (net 4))
 (segment (start 284.5 80.29) (end 287.59 77.2) (width 0.2) (layer "F.Cu") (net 4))
 (segment (start 172.001 19.632529) (end 172.001 26.9081) (width 0.2) (layer "F.Cu") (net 4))
 (segment (start 103.69 44.06) (end 103.69 67.065) (width 0.2) (layer "F.Cu") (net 15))
 (segment (start 103.69 67.065) (end 115.695 79.07) (width 0.2) (layer "F.Cu") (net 15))
 (segment (start 144.59 92.67) (end 137.32 99.94) (width 0.2) (layer "F.Cu") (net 11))
 (segment (start 144.59 91.23) (end 144.59 92.67) (width 0.2) (layer "F.Cu") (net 11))
 (via (at 137.32 99.94) (size 0.6) (drill 0.3) (layers "F.Cu" "B.Cu") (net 11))
 (via blind (at 144.59 91.23) (size 0.6) (drill 0.3) (layers "F.Cu" "B.Cu") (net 11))
 (segment (start 152.609 99.249) (end 144.59 91.23) (width 0.2) (layer "B.Cu") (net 11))
 (segment (start 137.32 96.210057) (end 120.179943 79.07) (width 0.2) (layer "B.Cu") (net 11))
 (segment (start 120.179943 79.07) (end 118.235 79.07) (width 0.2) (layer "B.Cu") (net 11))
 (segment (start 137.32 99.94) (end 137.32 96.210057) (width 0.2) (layer "B.Cu") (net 11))
 (segment (start 202.229 99.249) (end 152.609 99.249) (width 0.2) (layer "B.Cu") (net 11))
 (segment (start 217.63 114.65) (end 202.229 99.249) (width 0.2) (layer "B.Cu") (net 11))
 (segment (start 218.78 116.04) (end 220.17 114.65) (width 0.2) (layer "F.Cu") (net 6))
 (segment (start 177.25 116.04) (end 218.78 116.04) (width 0.2) (layer "F.Cu") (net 6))
 (segment (start 167.5 106.29) (end 177.25 116.04) (width 0.2) (layer "F.Cu") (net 6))
 (via (at 167.5 106.29) (size 0.6) (drill 0.3) (layers "F.Cu" "B.Cu") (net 6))
 (segment (start 141.479 74.431) (end 141.479 99.8161) (width 0.2) (layer "B.Cu") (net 6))
 (segment (start 156.12 59.79) (end 141.479 74.431) (width 0.2) (layer "B.Cu") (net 6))
 (segment (start 141.479 99.8161) (end 147.9529 106.29) (width 0.2) (layer "B.Cu") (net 6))
 (segment (start 147.9529 106.29) (end 167.5 106.29) (width 0.2) (layer "B.Cu") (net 6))
 (segment (start 162.3 42.39) (end 162.3 56.15) (width 0.2) (layer "F.Cu") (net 5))
 (segment (start 162.3 56.15) (end 158.66 59.79) (width 0.2) (layer "F.Cu") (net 5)))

